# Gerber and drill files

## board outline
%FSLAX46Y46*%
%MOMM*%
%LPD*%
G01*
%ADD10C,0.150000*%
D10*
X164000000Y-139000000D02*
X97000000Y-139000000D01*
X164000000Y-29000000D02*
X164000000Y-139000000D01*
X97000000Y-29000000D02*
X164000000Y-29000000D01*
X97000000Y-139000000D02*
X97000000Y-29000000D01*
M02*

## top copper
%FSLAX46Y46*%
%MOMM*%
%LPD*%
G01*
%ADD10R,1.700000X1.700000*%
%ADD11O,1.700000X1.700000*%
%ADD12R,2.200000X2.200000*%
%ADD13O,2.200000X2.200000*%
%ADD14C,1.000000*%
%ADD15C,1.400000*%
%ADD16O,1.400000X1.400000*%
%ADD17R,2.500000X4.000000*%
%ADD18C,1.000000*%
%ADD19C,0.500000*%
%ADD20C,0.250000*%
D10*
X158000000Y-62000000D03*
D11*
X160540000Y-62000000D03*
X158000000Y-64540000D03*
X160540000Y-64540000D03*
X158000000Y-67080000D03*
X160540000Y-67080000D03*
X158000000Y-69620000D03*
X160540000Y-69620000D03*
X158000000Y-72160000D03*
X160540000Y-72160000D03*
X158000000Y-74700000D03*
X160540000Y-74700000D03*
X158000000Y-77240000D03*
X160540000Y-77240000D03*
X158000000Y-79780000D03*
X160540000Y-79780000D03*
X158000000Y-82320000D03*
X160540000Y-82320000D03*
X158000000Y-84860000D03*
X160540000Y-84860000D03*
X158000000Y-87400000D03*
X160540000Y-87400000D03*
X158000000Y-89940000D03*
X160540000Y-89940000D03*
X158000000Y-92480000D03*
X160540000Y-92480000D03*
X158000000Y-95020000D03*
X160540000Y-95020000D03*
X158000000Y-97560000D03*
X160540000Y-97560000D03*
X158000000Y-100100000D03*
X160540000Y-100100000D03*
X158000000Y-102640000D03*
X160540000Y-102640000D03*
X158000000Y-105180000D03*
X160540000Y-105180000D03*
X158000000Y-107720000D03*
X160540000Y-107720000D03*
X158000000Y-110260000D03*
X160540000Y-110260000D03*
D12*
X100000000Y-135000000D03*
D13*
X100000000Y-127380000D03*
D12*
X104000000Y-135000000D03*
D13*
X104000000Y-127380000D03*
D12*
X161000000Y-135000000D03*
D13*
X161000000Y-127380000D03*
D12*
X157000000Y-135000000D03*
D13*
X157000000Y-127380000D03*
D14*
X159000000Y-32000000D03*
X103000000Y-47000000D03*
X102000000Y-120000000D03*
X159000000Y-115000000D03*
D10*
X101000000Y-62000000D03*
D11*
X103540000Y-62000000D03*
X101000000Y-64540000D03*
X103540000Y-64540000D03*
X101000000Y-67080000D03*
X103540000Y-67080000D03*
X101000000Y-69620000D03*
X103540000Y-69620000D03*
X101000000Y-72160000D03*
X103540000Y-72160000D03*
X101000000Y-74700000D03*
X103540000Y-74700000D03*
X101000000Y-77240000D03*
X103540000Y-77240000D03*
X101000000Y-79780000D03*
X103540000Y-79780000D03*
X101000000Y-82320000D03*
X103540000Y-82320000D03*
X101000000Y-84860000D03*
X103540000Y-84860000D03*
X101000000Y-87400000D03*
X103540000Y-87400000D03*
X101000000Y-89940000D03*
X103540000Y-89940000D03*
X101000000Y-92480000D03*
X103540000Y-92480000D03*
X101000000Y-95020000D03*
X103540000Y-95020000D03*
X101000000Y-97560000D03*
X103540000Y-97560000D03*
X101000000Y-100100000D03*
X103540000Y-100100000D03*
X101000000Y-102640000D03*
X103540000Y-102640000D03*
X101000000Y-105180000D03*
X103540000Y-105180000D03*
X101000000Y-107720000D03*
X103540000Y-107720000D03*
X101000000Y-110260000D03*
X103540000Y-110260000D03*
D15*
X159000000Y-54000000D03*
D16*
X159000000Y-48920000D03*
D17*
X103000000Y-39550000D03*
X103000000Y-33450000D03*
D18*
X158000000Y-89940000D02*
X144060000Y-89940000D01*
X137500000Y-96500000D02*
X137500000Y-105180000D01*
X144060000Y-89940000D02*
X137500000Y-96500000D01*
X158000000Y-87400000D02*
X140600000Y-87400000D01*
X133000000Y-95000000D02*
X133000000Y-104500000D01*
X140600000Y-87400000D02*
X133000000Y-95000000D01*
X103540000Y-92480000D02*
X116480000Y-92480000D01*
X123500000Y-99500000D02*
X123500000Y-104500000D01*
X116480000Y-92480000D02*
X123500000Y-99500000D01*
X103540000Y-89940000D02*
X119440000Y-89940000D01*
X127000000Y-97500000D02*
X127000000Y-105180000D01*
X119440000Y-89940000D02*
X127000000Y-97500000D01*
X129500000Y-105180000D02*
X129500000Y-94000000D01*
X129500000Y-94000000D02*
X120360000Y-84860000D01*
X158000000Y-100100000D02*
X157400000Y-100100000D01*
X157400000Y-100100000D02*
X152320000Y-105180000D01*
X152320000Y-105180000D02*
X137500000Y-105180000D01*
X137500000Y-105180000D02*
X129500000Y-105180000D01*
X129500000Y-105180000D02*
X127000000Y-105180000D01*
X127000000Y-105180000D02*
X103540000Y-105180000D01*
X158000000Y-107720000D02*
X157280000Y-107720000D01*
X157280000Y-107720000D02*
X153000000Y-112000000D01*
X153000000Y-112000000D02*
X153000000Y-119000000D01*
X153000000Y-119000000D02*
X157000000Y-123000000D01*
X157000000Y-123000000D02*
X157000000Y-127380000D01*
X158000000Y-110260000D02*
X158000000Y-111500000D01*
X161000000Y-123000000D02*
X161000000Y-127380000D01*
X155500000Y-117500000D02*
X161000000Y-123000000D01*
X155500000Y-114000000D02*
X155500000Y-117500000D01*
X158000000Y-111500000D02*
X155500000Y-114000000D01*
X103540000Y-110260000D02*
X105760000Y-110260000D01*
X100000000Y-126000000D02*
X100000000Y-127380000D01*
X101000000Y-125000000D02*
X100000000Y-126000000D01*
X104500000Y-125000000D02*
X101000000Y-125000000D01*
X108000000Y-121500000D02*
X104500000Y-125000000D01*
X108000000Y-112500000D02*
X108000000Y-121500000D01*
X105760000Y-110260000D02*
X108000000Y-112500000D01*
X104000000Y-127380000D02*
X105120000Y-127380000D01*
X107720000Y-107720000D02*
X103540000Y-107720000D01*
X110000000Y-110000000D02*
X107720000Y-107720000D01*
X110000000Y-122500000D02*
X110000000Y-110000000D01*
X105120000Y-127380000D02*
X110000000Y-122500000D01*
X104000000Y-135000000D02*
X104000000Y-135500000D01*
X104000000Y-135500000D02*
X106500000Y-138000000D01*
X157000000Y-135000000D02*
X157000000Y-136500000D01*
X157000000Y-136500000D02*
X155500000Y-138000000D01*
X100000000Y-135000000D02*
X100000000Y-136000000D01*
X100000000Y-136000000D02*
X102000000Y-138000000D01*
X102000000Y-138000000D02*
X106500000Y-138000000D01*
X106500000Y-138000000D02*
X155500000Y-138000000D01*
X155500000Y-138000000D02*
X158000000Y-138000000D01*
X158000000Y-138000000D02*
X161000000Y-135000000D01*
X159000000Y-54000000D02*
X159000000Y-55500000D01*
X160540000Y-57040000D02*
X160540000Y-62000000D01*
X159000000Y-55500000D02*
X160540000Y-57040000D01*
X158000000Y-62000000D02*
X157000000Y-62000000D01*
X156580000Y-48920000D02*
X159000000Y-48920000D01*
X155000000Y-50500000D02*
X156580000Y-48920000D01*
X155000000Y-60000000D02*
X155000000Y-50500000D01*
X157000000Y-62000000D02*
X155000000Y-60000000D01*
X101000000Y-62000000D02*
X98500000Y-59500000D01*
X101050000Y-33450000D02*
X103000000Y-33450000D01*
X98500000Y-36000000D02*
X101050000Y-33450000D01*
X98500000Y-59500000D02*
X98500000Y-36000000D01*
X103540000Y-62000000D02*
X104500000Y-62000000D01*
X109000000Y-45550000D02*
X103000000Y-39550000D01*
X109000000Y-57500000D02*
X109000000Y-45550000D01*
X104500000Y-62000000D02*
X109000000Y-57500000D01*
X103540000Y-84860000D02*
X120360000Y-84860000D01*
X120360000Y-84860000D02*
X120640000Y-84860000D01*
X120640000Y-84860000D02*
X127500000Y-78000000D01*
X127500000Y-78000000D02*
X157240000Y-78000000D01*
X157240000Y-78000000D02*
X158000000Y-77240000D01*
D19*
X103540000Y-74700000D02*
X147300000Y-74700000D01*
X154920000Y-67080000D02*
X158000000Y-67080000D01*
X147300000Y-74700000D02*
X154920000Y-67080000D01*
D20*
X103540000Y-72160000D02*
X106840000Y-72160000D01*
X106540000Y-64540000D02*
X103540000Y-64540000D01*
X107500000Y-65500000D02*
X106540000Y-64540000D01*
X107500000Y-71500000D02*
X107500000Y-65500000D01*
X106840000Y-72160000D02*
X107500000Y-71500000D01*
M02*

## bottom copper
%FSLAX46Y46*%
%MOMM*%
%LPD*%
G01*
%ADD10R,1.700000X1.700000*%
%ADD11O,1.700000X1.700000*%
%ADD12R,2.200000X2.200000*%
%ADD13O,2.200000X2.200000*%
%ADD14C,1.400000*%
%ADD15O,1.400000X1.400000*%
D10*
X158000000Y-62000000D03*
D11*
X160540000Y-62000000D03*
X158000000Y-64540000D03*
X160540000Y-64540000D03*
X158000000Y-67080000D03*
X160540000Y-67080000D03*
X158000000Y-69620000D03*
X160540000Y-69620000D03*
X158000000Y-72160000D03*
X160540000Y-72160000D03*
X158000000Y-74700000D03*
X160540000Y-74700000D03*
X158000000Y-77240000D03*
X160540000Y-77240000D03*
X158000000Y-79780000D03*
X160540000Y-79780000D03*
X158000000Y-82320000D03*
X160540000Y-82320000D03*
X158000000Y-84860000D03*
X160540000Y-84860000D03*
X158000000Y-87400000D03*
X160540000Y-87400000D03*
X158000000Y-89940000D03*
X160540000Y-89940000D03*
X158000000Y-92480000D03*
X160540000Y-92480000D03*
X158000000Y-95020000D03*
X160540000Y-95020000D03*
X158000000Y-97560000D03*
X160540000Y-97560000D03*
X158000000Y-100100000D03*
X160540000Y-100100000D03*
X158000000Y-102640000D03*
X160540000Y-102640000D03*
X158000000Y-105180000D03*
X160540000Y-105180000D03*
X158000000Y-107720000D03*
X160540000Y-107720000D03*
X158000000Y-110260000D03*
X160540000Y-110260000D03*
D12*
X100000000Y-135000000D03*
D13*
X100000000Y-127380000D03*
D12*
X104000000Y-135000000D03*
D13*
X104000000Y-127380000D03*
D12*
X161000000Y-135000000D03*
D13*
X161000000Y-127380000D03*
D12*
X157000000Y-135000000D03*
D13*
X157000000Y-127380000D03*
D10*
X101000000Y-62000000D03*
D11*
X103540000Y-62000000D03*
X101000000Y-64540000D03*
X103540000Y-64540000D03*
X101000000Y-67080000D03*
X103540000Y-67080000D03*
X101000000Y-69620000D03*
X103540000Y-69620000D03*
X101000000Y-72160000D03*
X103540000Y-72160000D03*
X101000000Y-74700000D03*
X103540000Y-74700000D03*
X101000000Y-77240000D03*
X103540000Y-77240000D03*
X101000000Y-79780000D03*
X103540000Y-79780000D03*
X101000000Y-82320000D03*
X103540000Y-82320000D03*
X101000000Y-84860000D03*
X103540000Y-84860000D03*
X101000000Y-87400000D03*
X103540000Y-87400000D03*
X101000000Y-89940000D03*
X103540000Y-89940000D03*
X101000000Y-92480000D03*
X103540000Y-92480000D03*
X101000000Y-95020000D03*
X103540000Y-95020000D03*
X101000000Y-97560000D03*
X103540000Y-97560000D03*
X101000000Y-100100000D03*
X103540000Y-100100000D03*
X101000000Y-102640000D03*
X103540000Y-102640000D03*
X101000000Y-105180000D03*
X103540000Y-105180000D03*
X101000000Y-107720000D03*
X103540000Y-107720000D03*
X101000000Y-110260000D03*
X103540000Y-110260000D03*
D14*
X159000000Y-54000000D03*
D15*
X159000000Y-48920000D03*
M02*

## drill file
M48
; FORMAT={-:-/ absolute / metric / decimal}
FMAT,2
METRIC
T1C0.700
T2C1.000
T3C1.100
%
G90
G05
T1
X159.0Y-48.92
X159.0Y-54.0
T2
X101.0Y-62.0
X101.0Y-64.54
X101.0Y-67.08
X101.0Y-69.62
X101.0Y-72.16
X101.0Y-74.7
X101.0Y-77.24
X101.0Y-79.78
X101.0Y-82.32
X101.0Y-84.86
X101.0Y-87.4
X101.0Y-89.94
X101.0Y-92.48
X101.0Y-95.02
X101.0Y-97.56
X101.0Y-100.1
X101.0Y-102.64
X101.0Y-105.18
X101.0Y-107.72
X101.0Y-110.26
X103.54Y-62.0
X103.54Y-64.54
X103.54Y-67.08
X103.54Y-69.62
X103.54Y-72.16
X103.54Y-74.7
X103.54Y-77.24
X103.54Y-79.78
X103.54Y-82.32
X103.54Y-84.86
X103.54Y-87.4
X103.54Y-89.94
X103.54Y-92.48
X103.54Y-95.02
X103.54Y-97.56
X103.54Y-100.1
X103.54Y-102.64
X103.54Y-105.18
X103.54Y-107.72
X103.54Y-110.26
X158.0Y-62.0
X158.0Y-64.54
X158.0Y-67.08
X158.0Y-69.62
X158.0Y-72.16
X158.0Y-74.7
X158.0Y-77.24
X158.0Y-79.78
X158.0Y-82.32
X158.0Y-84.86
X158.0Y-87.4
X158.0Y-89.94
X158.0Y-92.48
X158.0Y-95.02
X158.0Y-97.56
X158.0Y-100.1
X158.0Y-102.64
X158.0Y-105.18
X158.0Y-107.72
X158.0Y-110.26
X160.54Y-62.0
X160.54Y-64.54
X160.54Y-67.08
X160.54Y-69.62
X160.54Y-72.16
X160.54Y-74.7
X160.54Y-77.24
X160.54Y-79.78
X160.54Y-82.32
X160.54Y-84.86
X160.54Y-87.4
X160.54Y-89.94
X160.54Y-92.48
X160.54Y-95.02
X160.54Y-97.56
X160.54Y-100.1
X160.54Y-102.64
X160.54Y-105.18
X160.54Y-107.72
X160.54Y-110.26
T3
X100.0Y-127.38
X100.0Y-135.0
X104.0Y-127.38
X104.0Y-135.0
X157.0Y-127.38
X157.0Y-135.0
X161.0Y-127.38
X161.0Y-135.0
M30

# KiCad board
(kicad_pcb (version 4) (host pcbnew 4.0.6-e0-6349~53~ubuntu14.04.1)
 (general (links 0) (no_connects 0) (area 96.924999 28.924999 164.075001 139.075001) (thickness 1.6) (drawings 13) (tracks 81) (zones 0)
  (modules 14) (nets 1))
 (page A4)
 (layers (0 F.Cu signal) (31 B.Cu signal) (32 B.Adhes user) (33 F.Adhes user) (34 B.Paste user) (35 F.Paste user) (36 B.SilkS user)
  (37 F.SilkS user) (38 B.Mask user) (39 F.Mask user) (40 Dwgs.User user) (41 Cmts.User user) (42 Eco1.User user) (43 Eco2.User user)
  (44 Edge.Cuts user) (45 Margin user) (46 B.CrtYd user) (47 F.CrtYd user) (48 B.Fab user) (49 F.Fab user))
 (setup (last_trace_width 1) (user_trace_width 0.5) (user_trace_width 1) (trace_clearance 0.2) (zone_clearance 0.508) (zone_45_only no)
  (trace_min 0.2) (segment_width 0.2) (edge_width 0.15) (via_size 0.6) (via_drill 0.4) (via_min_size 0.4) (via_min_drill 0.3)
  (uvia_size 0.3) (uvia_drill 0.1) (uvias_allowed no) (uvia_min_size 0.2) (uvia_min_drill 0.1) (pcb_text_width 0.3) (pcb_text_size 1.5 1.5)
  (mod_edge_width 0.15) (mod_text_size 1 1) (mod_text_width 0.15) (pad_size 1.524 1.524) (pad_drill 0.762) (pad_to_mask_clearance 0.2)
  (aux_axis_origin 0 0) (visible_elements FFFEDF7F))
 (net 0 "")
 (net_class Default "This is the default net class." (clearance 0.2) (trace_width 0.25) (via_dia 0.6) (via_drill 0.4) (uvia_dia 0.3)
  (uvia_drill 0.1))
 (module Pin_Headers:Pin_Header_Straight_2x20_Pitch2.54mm (layer F.Cu) (at 158 62)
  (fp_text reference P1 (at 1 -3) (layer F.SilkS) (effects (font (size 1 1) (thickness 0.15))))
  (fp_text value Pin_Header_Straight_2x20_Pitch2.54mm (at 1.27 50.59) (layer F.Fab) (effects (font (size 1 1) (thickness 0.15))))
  (pad 1 thru_hole rect (at 0 0) (size 1.7 1.7) (drill 1) (layers *.Cu *.Mask))
  (pad 2 thru_hole oval (at 2.54 0) (size 1.7 1.7) (drill 1) (layers *.Cu *.Mask))
  (pad 3 thru_hole oval (at 0 2.54) (size 1.7 1.7) (drill 1) (layers *.Cu *.Mask))
  (pad 4 thru_hole oval (at 2.54 2.54) (size 1.7 1.7) (drill 1) (layers *.Cu *.Mask))
  (pad 5 thru_hole oval (at 0 5.08) (size 1.7 1.7) (drill 1) (layers *.Cu *.Mask))
  (pad 6 thru_hole oval (at 2.54 5.08) (size 1.7 1.7) (drill 1) (layers *.Cu *.Mask))
  (pad 7 thru_hole oval (at 0 7.62) (size 1.7 1.7) (drill 1) (layers *.Cu *.Mask))
  (pad 8 thru_hole oval (at 2.54 7.62) (size 1.7 1.7) (drill 1) (layers *.Cu *.Mask))
  (pad 9 thru_hole oval (at 0 10.16) (size 1.7 1.7) (drill 1) (layers *.Cu *.Mask))
  (pad 10 thru_hole oval (at 2.54 10.16) (size 1.7 1.7) (drill 1) (layers *.Cu *.Mask))
  (pad 11 thru_hole oval (at 0 12.7) (size 1.7 1.7) (drill 1) (layers *.Cu *.Mask))
  (pad 12 thru_hole oval (at 2.54 12.7) (size 1.7 1.7) (drill 1) (layers *.Cu *.Mask))
  (pad 13 thru_hole oval (at 0 15.24) (size 1.7 1.7) (drill 1) (layers *.Cu *.Mask))
  (pad 14 thru_hole oval (at 2.54 15.24) (size 1.7 1.7) (drill 1) (layers *.Cu *.Mask))
  (pad 15 thru_hole oval (at 0 17.78) (size 1.7 1.7) (drill 1) (layers *.Cu *.Mask))
  (pad 16 thru_hole oval (at 2.54 17.78) (size 1.7 1.7) (drill 1) (layers *.Cu *.Mask))
  (pad 17 thru_hole oval (at 0 20.32) (size 1.7 1.7) (drill 1) (layers *.Cu *.Mask))
  (pad 18 thru_hole oval (at 2.54 20.32) (size 1.7 1.7) (drill 1) (layers *.Cu *.Mask))
  (pad 19 thru_hole oval (at 0 22.86) (size 1.7 1.7) (drill 1) (layers *.Cu *.Mask))
  (pad 20 thru_hole oval (at 2.54 22.86) (size 1.7 1.7) (drill 1) (layers *.Cu *.Mask))
  (pad 21 thru_hole oval (at 0 25.4) (size 1.7 1.7) (drill 1) (layers *.Cu *.Mask))
  (pad 22 thru_hole oval (at 2.54 25.4) (size 1.7 1.7) (drill 1) (layers *.Cu *.Mask))
  (pad 23 thru_hole oval (at 0 27.94) (size 1.7 1.7) (drill 1) (layers *.Cu *.Mask))
  (pad 24 thru_hole oval (at 2.54 27.94) (size 1.7 1.7) (drill 1) (layers *.Cu *.Mask))
  (pad 25 thru_hole oval (at 0 30.48) (size 1.7 1.7) (drill 1) (layers *.Cu *.Mask))
  (pad 26 thru_hole oval (at 2.54 30.48) (size 1.7 1.7) (drill 1) (layers *.Cu *.Mask))
  (pad 27 thru_hole oval (at 0 33.02) (size 1.7 1.7) (drill 1) (layers *.Cu *.Mask))
  (pad 28 thru_hole oval (at 2.54 33.02) (size 1.7 1.7) (drill 1) (layers *.Cu *.Mask))
  (pad 29 thru_hole oval (at 0 35.56) (size 1.7 1.7) (drill 1) (layers *.Cu *.Mask))
  (pad 30 thru_hole oval (at 2.54 35.56) (size 1.7 1.7) (drill 1) (layers *.Cu *.Mask))
  (pad 31 thru_hole oval (at 0 38.1) (size 1.7 1.7) (drill 1) (layers *.Cu *.Mask))
  (pad 32 thru_hole oval (at 2.54 38.1) (size 1.7 1.7) (drill 1) (layers *.Cu *.Mask))
  (pad 33 thru_hole oval (at 0 40.64) (size 1.7 1.7) (drill 1) (layers *.Cu *.Mask))
  (pad 34 thru_hole oval (at 2.54 40.64) (size 1.7 1.7) (drill 1) (layers *.Cu *.Mask))
  (pad 35 thru_hole oval (at 0 43.18) (size 1.7 1.7) (drill 1) (layers *.Cu *.Mask))
  (pad 36 thru_hole oval (at 2.54 43.18) (size 1.7 1.7) (drill 1) (layers *.Cu *.Mask))
  (pad 37 thru_hole oval (at 0 45.72) (size 1.7 1.7) (drill 1) (layers *.Cu *.Mask))
  (pad 38 thru_hole oval (at 2.54 45.72) (size 1.7 1.7) (drill 1) (layers *.Cu *.Mask))
  (pad 39 thru_hole oval (at 0 48.26) (size 1.7 1.7) (drill 1) (layers *.Cu *.Mask))
  (pad 40 thru_hole oval (at 2.54 48.26) (size 1.7 1.7) (drill 1) (layers *.Cu *.Mask)))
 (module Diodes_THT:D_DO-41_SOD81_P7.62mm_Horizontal (layer F.Cu) (at 100 135 90)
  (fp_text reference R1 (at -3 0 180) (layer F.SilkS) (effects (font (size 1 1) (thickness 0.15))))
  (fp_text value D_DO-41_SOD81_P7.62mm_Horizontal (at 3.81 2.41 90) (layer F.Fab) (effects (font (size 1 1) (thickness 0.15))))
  (pad 1 thru_hole rect (at 0 0 90) (size 2.2 2.2) (drill 1.1) (layers *.Cu *.Mask))
  (pad 2 thru_hole oval (at 7.62 0 90) (size 2.2 2.2) (drill 1.1) (layers *.Cu *.Mask)))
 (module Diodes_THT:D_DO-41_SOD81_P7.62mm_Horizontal (layer F.Cu) (at 104 135 90)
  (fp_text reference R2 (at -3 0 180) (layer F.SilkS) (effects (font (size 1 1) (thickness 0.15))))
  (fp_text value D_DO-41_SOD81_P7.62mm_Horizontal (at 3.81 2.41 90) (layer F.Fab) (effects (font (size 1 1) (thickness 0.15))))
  (pad 1 thru_hole rect (at 0 0 90) (size 2.2 2.2) (drill 1.1) (layers *.Cu *.Mask))
  (pad 2 thru_hole oval (at 7.62 0 90) (size 2.2 2.2) (drill 1.1) (layers *.Cu *.Mask)))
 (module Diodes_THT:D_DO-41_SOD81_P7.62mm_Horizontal (layer F.Cu) (at 161 135 90)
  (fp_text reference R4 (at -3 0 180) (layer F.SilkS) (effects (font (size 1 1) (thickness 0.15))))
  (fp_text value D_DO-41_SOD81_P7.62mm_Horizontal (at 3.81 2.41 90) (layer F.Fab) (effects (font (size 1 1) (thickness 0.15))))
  (pad 1 thru_hole rect (at 0 0 90) (size 2.2 2.2) (drill 1.1) (layers *.Cu *.Mask))
  (pad 2 thru_hole oval (at 7.62 0 90) (size 2.2 2.2) (drill 1.1) (layers *.Cu *.Mask)))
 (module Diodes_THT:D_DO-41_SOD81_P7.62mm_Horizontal (layer F.Cu) (at 157 135 90)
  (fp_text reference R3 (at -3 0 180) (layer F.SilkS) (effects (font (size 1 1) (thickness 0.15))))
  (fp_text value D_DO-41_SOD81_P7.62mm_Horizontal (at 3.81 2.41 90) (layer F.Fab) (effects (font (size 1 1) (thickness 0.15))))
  (pad 1 thru_hole rect (at 0 0 90) (size 2.2 2.2) (drill 1.1) (layers *.Cu *.Mask))
  (pad 2 thru_hole oval (at 7.62 0 90) (size 2.2 2.2) (drill 1.1) (layers *.Cu *.Mask)))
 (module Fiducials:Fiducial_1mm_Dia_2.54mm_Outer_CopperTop (layer F.Cu) (at 159 32)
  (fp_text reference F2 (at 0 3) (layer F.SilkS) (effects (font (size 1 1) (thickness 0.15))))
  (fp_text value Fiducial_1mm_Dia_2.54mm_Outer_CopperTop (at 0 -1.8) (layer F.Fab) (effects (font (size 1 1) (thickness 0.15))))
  (pad ~ smd circle (at 0 0) (size 1 1) (layers F.Cu F.Mask) (solder_mask_margin 0.77) (clearance 0.77)))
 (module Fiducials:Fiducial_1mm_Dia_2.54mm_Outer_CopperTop (layer F.Cu) (at 103 47)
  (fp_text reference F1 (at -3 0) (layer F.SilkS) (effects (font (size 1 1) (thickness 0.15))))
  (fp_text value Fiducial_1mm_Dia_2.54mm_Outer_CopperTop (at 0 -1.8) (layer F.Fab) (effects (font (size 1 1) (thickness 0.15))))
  (pad ~ smd circle (at 0 0) (size 1 1) (layers F.Cu F.Mask) (solder_mask_margin 0.77) (clearance 0.77)))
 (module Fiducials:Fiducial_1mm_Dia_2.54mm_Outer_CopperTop (layer F.Cu) (at 102 120)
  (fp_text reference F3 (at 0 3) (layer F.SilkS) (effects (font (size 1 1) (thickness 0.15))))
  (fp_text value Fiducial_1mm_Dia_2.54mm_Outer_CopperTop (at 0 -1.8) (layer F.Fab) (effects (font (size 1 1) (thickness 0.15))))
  (pad ~ smd circle (at 0 0) (size 1 1) (layers F.Cu F.Mask) (solder_mask_margin 0.77) (clearance 0.77)))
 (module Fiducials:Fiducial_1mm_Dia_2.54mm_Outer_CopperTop (layer F.Cu) (at 159 115)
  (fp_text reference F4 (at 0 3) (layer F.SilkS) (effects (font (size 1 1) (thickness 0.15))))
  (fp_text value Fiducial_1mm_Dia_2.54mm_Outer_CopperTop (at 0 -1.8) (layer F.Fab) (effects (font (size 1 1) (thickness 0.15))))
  (pad ~ smd circle (at 0 0) (size 1 1) (layers F.Cu F.Mask) (solder_mask_margin 0.77) (clearance 0.77)))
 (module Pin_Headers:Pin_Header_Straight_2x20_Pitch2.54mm (layer F.Cu) (at 101 62)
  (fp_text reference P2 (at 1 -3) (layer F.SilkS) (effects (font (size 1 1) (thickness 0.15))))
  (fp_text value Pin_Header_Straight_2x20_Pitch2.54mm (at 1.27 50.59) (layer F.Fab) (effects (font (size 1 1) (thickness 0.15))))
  (pad 1 thru_hole rect (at 0 0) (size 1.7 1.7) (drill 1) (layers *.Cu *.Mask))
  (pad 2 thru_hole oval (at 2.54 0) (size 1.7 1.7) (drill 1) (layers *.Cu *.Mask))
  (pad 3 thru_hole oval (at 0 2.54) (size 1.7 1.7) (drill 1) (layers *.Cu *.Mask))
  (pad 4 thru_hole oval (at 2.54 2.54) (size 1.7 1.7) (drill 1) (layers *.Cu *.Mask))
  (pad 5 thru_hole oval (at 0 5.08) (size 1.7 1.7) (drill 1) (layers *.Cu *.Mask))
  (pad 6 thru_hole oval (at 2.54 5.08) (size 1.7 1.7) (drill 1) (layers *.Cu *.Mask))
  (pad 7 thru_hole oval (at 0 7.62) (size 1.7 1.7) (drill 1) (layers *.Cu *.Mask))
  (pad 8 thru_hole oval (at 2.54 7.62) (size 1.7 1.7) (drill 1) (layers *.Cu *.Mask))
  (pad 9 thru_hole oval (at 0 10.16) (size 1.7 1.7) (drill 1) (layers *.Cu *.Mask))
  (pad 10 thru_hole oval (at 2.54 10.16) (size 1.7 1.7) (drill 1) (layers *.Cu *.Mask))
  (pad 11 thru_hole oval (at 0 12.7) (size 1.7 1.7) (drill 1) (layers *.Cu *.Mask))
  (pad 12 thru_hole oval (at 2.54 12.7) (size 1.7 1.7) (drill 1) (layers *.Cu *.Mask))
  (pad 13 thru_hole oval (at 0 15.24) (size 1.7 1.7) (drill 1) (layers *.Cu *.Mask))
  (pad 14 thru_hole oval (at 2.54 15.24) (size 1.7 1.7) (drill 1) (layers *.Cu *.Mask))
  (pad 15 thru_hole oval (at 0 17.78) (size 1.7 1.7) (drill 1) (layers *.Cu *.Mask))
  (pad 16 thru_hole oval (at 2.54 17.78) (size 1.7 1.7) (drill 1) (layers *.Cu *.Mask))
  (pad 17 thru_hole oval (at 0 20.32) (size 1.7 1.7) (drill 1) (layers *.Cu *.Mask))
  (pad 18 thru_hole oval (at 2.54 20.32) (size 1.7 1.7) (drill 1) (layers *.Cu *.Mask))
  (pad 19 thru_hole oval (at 0 22.86) (size 1.7 1.7) (drill 1) (layers *.Cu *.Mask))
  (pad 20 thru_hole oval (at 2.54 22.86) (size 1.7 1.7) (drill 1) (layers *.Cu *.Mask))
  (pad 21 thru_hole oval (at 0 25.4) (size 1.7 1.7) (drill 1) (layers *.Cu *.Mask))
  (pad 22 thru_hole oval (at 2.54 25.4) (size 1.7 1.7) (drill 1) (layers *.Cu *.Mask))
  (pad 23 thru_hole oval (at 0 27.94) (size 1.7 1.7) (drill 1) (layers *.Cu *.Mask))
  (pad 24 thru_hole oval (at 2.54 27.94) (size 1.7 1.7) (drill 1) (layers *.Cu *.Mask))
  (pad 25 thru_hole oval (at 0 30.48) (size 1.7 1.7) (drill 1) (layers *.Cu *.Mask))
  (pad 26 thru_hole oval (at 2.54 30.48) (size 1.7 1.7) (drill 1) (layers *.Cu *.Mask))
  (pad 27 thru_hole oval (at 0 33.02) (size 1.7 1.7) (drill 1) (layers *.Cu *.Mask))
  (pad 28 thru_hole oval (at 2.54 33.02) (size 1.7 1.7) (drill 1) (layers *.Cu *.Mask))
  (pad 29 thru_hole oval (at 0 35.56) (size 1.7 1.7) (drill 1) (layers *.Cu *.Mask))
  (pad 30 thru_hole oval (at 2.54 35.56) (size 1.7 1.7) (drill 1) (layers *.Cu *.Mask))
  (pad 31 thru_hole oval (at 0 38.1) (size 1.7 1.7) (drill 1) (layers *.Cu *.Mask))
  (pad 32 thru_hole oval (at 2.54 38.1) (size 1.7 1.7) (drill 1) (layers *.Cu *.Mask))
  (pad 33 thru_hole oval (at 0 40.64) (size 1.7 1.7) (drill 1) (layers *.Cu *.Mask))
  (pad 34 thru_hole oval (at 2.54 40.64) (size 1.7 1.7) (drill 1) (layers *.Cu *.Mask))
  (pad 35 thru_hole oval (at 0 43.18) (size 1.7 1.7) (drill 1) (layers *.Cu *.Mask))
  (pad 36 thru_hole oval (at 2.54 43.18) (size 1.7 1.7) (drill 1) (layers *.Cu *.Mask))
  (pad 37 thru_hole oval (at 0 45.72) (size 1.7 1.7) (drill 1) (layers *.Cu *.Mask))
  (pad 38 thru_hole oval (at 2.54 45.72) (size 1.7 1.7) (drill 1) (layers *.Cu *.Mask))
  (pad 39 thru_hole oval (at 0 48.26) (size 1.7 1.7) (drill 1) (layers *.Cu *.Mask))
  (pad 40 thru_hole oval (at 2.54 48.26) (size 1.7 1.7) (drill 1) (layers *.Cu *.Mask)))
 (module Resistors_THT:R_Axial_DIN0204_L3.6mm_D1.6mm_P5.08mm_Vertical (layer F.Cu) (at 159 54 90)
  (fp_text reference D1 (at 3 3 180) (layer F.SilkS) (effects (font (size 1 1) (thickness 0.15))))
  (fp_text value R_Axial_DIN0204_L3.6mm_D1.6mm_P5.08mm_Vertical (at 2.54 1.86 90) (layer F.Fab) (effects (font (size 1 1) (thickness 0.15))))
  (pad 1 thru_hole circle (at 0 0 90) (size 1.4 1.4) (drill 0.7) (layers *.Cu *.Mask))
  (pad 2 thru_hole oval (at 5.08 0 90) (size 1.4 1.4) (drill 0.7) (layers *.Cu *.Mask)))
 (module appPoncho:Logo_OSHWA (layer F.Cu) (at 159 41)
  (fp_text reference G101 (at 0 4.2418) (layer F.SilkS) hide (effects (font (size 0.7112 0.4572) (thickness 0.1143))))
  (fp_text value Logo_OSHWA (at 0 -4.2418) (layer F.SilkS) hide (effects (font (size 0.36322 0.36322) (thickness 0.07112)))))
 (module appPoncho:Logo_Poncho (layer F.Cu) (at 131 35.5)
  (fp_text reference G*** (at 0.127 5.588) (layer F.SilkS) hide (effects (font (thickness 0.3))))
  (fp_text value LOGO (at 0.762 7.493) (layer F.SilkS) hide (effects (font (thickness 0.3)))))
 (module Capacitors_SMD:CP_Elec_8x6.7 (layer F.Cu) (at 103 36.5 90)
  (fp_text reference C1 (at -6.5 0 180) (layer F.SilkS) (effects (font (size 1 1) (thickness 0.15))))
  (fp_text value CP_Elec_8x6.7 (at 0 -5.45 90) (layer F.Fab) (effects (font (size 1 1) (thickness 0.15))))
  (pad 1 smd rect (at -3.05 0 270) (size 4 2.5) (layers F.Cu F.Paste F.Mask))
  (pad 2 smd rect (at 3.05 0 270) (size 4 2.5) (layers F.Cu F.Paste F.Mask)))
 (gr_line (start 164 139) (end 97 139) (angle 90) (layer Edge.Cuts) (width 0.15))
 (gr_line (start 164 29) (end 164 139) (angle 90) (layer Edge.Cuts) (width 0.15))
 (gr_line (start 97 29) (end 164 29) (angle 90) (layer Edge.Cuts) (width 0.15))
 (gr_line (start 97 139) (end 97 29) (angle 90) (layer Edge.Cuts) (width 0.15))
 (segment (start 158 89.94) (end 144.06 89.94) (width 1) (layer F.Cu) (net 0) (status 400000))
 (segment (start 137.5 96.5) (end 137.5 105.18) (width 1) (layer F.Cu) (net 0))
 (segment (start 144.06 89.94) (end 137.5 96.5) (width 1) (layer F.Cu) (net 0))
 (segment (start 158 87.4) (end 140.6 87.4) (width 1) (layer F.Cu) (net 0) (status 400000))
 (segment (start 133 95) (end 133 104.5) (width 1) (layer F.Cu) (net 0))
 (segment (start 140.6 87.4) (end 133 95) (width 1) (layer F.Cu) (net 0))
 (segment (start 103.54 92.48) (end 116.48 92.48) (width 1) (layer F.Cu) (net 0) (status 400000))
 (segment (start 123.5 99.5) (end 123.5 104.5) (width 1) (layer F.Cu) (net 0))
 (segment (start 116.48 92.48) (end 123.5 99.5) (width 1) (layer F.Cu) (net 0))
 (segment (start 103.54 89.94) (end 119.44 89.94) (width 1) (layer F.Cu) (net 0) (status 400000))
 (segment (start 127 97.5) (end 127 105.18) (width 1) (layer F.Cu) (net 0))
 (segment (start 119.44 89.94) (end 127 97.5) (width 1) (layer F.Cu) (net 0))
 (segment (start 129.5 105.18) (end 129.5 94) (width 1) (layer F.Cu) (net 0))
 (segment (start 129.5 94) (end 120.36 84.86) (width 1) (layer F.Cu) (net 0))
 (segment (start 158 100.1) (end 157.4 100.1) (width 1) (layer F.Cu) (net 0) (status C00000))
 (segment (start 157.4 100.1) (end 152.32 105.18) (width 1) (layer F.Cu) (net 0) (status 400000))
 (segment (start 152.32 105.18) (end 137.5 105.18) (width 1) (layer F.Cu) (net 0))
 (segment (start 137.5 105.18) (end 129.5 105.18) (width 1) (layer F.Cu) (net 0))
 (segment (start 129.5 105.18) (end 127 105.18) (width 1) (layer F.Cu) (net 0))
 (segment (start 127 105.18) (end 103.54 105.18) (width 1) (layer F.Cu) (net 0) (status 800000))
 (segment (start 158 107.72) (end 157.28 107.72) (width 1) (layer F.Cu) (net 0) (status C00000))
 (segment (start 157.28 107.72) (end 153 112) (width 1) (layer F.Cu) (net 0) (status 400000))
 (segment (start 153 112) (end 153 119) (width 1) (layer F.Cu) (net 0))
 (segment (start 153 119) (end 157 123) (width 1) (layer F.Cu) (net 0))
 (segment (start 157 123) (end 157 127.38) (width 1) (layer F.Cu) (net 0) (status 800000))
 (segment (start 158 110.26) (end 158 111.5) (width 1) (layer F.Cu) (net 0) (status 400000))
 (segment (start 161 123) (end 161 127.38) (width 1) (layer F.Cu) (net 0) (status 800000))
 (segment (start 155.5 117.5) (end 161 123) (width 1) (layer F.Cu) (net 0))
 (segment (start 155.5 114) (end 155.5 117.5) (width 1) (layer F.Cu) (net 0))
 (segment (start 158 111.5) (end 155.5 114) (width 1) (layer F.Cu) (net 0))
 (segment (start 103.54 110.26) (end 105.76 110.26) (width 1) (layer F.Cu) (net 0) (status 400000))
 (segment (start 100 126) (end 100 127.38) (width 1) (layer F.Cu) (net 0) (status 800000))
 (segment (start 101 125) (end 100 126) (width 1) (layer F.Cu) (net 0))
 (segment (start 104.5 125) (end 101 125) (width 1) (layer F.Cu) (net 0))
 (segment (start 108 121.5) (end 104.5 125) (width 1) (layer F.Cu) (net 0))
 (segment (start 108 112.5) (end 108 121.5) (width 1) (layer F.Cu) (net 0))
 (segment (start 105.76 110.26) (end 108 112.5) (width 1) (layer F.Cu) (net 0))
 (segment (start 104 127.38) (end 105.12 127.38) (width 1) (layer F.Cu) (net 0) (status 400000))
 (segment (start 107.72 107.72) (end 103.54 107.72) (width 1) (layer F.Cu) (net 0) (status 800000))
 (segment (start 110 110) (end 107.72 107.72) (width 1) (layer F.Cu) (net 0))
 (segment (start 110 122.5) (end 110 110) (width 1) (layer F.Cu) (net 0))
 (segment (start 105.12 127.38) (end 110 122.5) (width 1) (layer F.Cu) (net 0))
 (segment (start 104 135) (end 104 135.5) (width 1) (layer F.Cu) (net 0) (status C00000))
 (segment (start 104 135.5) (end 106.5 138) (width 1) (layer F.Cu) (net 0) (status 400000))
 (segment (start 157 135) (end 157 136.5) (width 1) (layer F.Cu) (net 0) (status 400000))
 (segment (start 157 136.5) (end 155.5 138) (width 1) (layer F.Cu) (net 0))
 (segment (start 100 135) (end 100 136) (width 1) (layer F.Cu) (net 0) (status C00000))
 (segment (start 100 136) (end 102 138) (width 1) (layer F.Cu) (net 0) (status 400000))
 (segment (start 102 138) (end 106.5 138) (width 1) (layer F.Cu) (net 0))
 (segment (start 106.5 138) (end 155.5 138) (width 1) (layer F.Cu) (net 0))
 (segment (start 155.5 138) (end 158 138) (width 1) (layer F.Cu) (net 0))
 (segment (start 158 138) (end 161 135) (width 1) (layer F.Cu) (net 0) (status 800000))
 (segment (start 159 54) (end 159 55.5) (width 1) (layer F.Cu) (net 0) (status 400000))
 (segment (start 160.54 57.04) (end 160.54 62) (width 1) (layer F.Cu) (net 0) (status 800000))
 (segment (start 159 55.5) (end 160.54 57.04) (width 1) (layer F.Cu) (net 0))
 (segment (start 158 62) (end 157 62) (width 1) (layer F.Cu) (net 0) (status 400000))
 (segment (start 156.58 48.92) (end 159 48.92) (width 1) (layer F.Cu) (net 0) (status 800000))
 (segment (start 155 50.5) (end 156.58 48.92) (width 1) (layer F.Cu) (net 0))
 (segment (start 155 60) (end 155 50.5) (width 1) (layer F.Cu) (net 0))
 (segment (start 157 62) (end 155 60) (width 1) (layer F.Cu) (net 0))
 (segment (start 101 62) (end 98.5 59.5) (width 1) (layer F.Cu) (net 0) (status 400000))
 (segment (start 101.05 33.45) (end 103 33.45) (width 1) (layer F.Cu) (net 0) (status 800000))
 (segment (start 98.5 36) (end 101.05 33.45) (width 1) (layer F.Cu) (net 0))
 (segment (start 98.5 59.5) (end 98.5 36) (width 1) (layer F.Cu) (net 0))
 (segment (start 103.54 62) (end 104.5 62) (width 1) (layer F.Cu) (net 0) (status 400000))
 (segment (start 109 45.55) (end 103 39.55) (width 1) (layer F.Cu) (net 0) (status 800000))
 (segment (start 109 57.5) (end 109 45.55) (width 1) (layer F.Cu) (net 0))
 (segment (start 104.5 62) (end 109 57.5) (width 1) (layer F.Cu) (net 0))
 (segment (start 103.54 84.86) (end 120.36 84.86) (width 1) (layer F.Cu) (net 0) (status 400000))
 (segment (start 120.36 84.86) (end 120.64 84.86) (width 1) (layer F.Cu) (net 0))
 (segment (start 120.64 84.86) (end 127.5 78) (width 1) (layer F.Cu) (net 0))
 (segment (start 127.5 78) (end 157.24 78) (width 1) (layer F.Cu) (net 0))
 (segment (start 157.24 78) (end 158 77.24) (width 1) (layer F.Cu) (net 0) (status 800000))
 (segment (start 103.54 74.7) (end 147.3 74.7) (width 0.5) (layer F.Cu) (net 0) (status 400000))
 (segment (start 154.92 67.08) (end 158 67.08) (width 0.5) (layer F.Cu) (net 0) (status 800000))
 (segment (start 147.3 74.7) (end 154.92 67.08) (width 0.5) (layer F.Cu) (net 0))
 (segment (start 103.54 72.16) (end 106.84 72.16) (width 0.25) (layer F.Cu) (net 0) (status 400000))
 (segment (start 106.54 64.54) (end 103.54 64.54) (width 0.25) (layer F.Cu) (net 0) (status 800000))
 (segment (start 107.5 65.5) (end 106.54 64.54) (width 0.25) (layer F.Cu) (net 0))
 (segment (start 107.5 71.5) (end 107.5 65.5) (width 0.25) (layer F.Cu) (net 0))
 (segment (start 106.84 72.16) (end 107.5 71.5) (width 0.25) (layer F.Cu) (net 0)))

